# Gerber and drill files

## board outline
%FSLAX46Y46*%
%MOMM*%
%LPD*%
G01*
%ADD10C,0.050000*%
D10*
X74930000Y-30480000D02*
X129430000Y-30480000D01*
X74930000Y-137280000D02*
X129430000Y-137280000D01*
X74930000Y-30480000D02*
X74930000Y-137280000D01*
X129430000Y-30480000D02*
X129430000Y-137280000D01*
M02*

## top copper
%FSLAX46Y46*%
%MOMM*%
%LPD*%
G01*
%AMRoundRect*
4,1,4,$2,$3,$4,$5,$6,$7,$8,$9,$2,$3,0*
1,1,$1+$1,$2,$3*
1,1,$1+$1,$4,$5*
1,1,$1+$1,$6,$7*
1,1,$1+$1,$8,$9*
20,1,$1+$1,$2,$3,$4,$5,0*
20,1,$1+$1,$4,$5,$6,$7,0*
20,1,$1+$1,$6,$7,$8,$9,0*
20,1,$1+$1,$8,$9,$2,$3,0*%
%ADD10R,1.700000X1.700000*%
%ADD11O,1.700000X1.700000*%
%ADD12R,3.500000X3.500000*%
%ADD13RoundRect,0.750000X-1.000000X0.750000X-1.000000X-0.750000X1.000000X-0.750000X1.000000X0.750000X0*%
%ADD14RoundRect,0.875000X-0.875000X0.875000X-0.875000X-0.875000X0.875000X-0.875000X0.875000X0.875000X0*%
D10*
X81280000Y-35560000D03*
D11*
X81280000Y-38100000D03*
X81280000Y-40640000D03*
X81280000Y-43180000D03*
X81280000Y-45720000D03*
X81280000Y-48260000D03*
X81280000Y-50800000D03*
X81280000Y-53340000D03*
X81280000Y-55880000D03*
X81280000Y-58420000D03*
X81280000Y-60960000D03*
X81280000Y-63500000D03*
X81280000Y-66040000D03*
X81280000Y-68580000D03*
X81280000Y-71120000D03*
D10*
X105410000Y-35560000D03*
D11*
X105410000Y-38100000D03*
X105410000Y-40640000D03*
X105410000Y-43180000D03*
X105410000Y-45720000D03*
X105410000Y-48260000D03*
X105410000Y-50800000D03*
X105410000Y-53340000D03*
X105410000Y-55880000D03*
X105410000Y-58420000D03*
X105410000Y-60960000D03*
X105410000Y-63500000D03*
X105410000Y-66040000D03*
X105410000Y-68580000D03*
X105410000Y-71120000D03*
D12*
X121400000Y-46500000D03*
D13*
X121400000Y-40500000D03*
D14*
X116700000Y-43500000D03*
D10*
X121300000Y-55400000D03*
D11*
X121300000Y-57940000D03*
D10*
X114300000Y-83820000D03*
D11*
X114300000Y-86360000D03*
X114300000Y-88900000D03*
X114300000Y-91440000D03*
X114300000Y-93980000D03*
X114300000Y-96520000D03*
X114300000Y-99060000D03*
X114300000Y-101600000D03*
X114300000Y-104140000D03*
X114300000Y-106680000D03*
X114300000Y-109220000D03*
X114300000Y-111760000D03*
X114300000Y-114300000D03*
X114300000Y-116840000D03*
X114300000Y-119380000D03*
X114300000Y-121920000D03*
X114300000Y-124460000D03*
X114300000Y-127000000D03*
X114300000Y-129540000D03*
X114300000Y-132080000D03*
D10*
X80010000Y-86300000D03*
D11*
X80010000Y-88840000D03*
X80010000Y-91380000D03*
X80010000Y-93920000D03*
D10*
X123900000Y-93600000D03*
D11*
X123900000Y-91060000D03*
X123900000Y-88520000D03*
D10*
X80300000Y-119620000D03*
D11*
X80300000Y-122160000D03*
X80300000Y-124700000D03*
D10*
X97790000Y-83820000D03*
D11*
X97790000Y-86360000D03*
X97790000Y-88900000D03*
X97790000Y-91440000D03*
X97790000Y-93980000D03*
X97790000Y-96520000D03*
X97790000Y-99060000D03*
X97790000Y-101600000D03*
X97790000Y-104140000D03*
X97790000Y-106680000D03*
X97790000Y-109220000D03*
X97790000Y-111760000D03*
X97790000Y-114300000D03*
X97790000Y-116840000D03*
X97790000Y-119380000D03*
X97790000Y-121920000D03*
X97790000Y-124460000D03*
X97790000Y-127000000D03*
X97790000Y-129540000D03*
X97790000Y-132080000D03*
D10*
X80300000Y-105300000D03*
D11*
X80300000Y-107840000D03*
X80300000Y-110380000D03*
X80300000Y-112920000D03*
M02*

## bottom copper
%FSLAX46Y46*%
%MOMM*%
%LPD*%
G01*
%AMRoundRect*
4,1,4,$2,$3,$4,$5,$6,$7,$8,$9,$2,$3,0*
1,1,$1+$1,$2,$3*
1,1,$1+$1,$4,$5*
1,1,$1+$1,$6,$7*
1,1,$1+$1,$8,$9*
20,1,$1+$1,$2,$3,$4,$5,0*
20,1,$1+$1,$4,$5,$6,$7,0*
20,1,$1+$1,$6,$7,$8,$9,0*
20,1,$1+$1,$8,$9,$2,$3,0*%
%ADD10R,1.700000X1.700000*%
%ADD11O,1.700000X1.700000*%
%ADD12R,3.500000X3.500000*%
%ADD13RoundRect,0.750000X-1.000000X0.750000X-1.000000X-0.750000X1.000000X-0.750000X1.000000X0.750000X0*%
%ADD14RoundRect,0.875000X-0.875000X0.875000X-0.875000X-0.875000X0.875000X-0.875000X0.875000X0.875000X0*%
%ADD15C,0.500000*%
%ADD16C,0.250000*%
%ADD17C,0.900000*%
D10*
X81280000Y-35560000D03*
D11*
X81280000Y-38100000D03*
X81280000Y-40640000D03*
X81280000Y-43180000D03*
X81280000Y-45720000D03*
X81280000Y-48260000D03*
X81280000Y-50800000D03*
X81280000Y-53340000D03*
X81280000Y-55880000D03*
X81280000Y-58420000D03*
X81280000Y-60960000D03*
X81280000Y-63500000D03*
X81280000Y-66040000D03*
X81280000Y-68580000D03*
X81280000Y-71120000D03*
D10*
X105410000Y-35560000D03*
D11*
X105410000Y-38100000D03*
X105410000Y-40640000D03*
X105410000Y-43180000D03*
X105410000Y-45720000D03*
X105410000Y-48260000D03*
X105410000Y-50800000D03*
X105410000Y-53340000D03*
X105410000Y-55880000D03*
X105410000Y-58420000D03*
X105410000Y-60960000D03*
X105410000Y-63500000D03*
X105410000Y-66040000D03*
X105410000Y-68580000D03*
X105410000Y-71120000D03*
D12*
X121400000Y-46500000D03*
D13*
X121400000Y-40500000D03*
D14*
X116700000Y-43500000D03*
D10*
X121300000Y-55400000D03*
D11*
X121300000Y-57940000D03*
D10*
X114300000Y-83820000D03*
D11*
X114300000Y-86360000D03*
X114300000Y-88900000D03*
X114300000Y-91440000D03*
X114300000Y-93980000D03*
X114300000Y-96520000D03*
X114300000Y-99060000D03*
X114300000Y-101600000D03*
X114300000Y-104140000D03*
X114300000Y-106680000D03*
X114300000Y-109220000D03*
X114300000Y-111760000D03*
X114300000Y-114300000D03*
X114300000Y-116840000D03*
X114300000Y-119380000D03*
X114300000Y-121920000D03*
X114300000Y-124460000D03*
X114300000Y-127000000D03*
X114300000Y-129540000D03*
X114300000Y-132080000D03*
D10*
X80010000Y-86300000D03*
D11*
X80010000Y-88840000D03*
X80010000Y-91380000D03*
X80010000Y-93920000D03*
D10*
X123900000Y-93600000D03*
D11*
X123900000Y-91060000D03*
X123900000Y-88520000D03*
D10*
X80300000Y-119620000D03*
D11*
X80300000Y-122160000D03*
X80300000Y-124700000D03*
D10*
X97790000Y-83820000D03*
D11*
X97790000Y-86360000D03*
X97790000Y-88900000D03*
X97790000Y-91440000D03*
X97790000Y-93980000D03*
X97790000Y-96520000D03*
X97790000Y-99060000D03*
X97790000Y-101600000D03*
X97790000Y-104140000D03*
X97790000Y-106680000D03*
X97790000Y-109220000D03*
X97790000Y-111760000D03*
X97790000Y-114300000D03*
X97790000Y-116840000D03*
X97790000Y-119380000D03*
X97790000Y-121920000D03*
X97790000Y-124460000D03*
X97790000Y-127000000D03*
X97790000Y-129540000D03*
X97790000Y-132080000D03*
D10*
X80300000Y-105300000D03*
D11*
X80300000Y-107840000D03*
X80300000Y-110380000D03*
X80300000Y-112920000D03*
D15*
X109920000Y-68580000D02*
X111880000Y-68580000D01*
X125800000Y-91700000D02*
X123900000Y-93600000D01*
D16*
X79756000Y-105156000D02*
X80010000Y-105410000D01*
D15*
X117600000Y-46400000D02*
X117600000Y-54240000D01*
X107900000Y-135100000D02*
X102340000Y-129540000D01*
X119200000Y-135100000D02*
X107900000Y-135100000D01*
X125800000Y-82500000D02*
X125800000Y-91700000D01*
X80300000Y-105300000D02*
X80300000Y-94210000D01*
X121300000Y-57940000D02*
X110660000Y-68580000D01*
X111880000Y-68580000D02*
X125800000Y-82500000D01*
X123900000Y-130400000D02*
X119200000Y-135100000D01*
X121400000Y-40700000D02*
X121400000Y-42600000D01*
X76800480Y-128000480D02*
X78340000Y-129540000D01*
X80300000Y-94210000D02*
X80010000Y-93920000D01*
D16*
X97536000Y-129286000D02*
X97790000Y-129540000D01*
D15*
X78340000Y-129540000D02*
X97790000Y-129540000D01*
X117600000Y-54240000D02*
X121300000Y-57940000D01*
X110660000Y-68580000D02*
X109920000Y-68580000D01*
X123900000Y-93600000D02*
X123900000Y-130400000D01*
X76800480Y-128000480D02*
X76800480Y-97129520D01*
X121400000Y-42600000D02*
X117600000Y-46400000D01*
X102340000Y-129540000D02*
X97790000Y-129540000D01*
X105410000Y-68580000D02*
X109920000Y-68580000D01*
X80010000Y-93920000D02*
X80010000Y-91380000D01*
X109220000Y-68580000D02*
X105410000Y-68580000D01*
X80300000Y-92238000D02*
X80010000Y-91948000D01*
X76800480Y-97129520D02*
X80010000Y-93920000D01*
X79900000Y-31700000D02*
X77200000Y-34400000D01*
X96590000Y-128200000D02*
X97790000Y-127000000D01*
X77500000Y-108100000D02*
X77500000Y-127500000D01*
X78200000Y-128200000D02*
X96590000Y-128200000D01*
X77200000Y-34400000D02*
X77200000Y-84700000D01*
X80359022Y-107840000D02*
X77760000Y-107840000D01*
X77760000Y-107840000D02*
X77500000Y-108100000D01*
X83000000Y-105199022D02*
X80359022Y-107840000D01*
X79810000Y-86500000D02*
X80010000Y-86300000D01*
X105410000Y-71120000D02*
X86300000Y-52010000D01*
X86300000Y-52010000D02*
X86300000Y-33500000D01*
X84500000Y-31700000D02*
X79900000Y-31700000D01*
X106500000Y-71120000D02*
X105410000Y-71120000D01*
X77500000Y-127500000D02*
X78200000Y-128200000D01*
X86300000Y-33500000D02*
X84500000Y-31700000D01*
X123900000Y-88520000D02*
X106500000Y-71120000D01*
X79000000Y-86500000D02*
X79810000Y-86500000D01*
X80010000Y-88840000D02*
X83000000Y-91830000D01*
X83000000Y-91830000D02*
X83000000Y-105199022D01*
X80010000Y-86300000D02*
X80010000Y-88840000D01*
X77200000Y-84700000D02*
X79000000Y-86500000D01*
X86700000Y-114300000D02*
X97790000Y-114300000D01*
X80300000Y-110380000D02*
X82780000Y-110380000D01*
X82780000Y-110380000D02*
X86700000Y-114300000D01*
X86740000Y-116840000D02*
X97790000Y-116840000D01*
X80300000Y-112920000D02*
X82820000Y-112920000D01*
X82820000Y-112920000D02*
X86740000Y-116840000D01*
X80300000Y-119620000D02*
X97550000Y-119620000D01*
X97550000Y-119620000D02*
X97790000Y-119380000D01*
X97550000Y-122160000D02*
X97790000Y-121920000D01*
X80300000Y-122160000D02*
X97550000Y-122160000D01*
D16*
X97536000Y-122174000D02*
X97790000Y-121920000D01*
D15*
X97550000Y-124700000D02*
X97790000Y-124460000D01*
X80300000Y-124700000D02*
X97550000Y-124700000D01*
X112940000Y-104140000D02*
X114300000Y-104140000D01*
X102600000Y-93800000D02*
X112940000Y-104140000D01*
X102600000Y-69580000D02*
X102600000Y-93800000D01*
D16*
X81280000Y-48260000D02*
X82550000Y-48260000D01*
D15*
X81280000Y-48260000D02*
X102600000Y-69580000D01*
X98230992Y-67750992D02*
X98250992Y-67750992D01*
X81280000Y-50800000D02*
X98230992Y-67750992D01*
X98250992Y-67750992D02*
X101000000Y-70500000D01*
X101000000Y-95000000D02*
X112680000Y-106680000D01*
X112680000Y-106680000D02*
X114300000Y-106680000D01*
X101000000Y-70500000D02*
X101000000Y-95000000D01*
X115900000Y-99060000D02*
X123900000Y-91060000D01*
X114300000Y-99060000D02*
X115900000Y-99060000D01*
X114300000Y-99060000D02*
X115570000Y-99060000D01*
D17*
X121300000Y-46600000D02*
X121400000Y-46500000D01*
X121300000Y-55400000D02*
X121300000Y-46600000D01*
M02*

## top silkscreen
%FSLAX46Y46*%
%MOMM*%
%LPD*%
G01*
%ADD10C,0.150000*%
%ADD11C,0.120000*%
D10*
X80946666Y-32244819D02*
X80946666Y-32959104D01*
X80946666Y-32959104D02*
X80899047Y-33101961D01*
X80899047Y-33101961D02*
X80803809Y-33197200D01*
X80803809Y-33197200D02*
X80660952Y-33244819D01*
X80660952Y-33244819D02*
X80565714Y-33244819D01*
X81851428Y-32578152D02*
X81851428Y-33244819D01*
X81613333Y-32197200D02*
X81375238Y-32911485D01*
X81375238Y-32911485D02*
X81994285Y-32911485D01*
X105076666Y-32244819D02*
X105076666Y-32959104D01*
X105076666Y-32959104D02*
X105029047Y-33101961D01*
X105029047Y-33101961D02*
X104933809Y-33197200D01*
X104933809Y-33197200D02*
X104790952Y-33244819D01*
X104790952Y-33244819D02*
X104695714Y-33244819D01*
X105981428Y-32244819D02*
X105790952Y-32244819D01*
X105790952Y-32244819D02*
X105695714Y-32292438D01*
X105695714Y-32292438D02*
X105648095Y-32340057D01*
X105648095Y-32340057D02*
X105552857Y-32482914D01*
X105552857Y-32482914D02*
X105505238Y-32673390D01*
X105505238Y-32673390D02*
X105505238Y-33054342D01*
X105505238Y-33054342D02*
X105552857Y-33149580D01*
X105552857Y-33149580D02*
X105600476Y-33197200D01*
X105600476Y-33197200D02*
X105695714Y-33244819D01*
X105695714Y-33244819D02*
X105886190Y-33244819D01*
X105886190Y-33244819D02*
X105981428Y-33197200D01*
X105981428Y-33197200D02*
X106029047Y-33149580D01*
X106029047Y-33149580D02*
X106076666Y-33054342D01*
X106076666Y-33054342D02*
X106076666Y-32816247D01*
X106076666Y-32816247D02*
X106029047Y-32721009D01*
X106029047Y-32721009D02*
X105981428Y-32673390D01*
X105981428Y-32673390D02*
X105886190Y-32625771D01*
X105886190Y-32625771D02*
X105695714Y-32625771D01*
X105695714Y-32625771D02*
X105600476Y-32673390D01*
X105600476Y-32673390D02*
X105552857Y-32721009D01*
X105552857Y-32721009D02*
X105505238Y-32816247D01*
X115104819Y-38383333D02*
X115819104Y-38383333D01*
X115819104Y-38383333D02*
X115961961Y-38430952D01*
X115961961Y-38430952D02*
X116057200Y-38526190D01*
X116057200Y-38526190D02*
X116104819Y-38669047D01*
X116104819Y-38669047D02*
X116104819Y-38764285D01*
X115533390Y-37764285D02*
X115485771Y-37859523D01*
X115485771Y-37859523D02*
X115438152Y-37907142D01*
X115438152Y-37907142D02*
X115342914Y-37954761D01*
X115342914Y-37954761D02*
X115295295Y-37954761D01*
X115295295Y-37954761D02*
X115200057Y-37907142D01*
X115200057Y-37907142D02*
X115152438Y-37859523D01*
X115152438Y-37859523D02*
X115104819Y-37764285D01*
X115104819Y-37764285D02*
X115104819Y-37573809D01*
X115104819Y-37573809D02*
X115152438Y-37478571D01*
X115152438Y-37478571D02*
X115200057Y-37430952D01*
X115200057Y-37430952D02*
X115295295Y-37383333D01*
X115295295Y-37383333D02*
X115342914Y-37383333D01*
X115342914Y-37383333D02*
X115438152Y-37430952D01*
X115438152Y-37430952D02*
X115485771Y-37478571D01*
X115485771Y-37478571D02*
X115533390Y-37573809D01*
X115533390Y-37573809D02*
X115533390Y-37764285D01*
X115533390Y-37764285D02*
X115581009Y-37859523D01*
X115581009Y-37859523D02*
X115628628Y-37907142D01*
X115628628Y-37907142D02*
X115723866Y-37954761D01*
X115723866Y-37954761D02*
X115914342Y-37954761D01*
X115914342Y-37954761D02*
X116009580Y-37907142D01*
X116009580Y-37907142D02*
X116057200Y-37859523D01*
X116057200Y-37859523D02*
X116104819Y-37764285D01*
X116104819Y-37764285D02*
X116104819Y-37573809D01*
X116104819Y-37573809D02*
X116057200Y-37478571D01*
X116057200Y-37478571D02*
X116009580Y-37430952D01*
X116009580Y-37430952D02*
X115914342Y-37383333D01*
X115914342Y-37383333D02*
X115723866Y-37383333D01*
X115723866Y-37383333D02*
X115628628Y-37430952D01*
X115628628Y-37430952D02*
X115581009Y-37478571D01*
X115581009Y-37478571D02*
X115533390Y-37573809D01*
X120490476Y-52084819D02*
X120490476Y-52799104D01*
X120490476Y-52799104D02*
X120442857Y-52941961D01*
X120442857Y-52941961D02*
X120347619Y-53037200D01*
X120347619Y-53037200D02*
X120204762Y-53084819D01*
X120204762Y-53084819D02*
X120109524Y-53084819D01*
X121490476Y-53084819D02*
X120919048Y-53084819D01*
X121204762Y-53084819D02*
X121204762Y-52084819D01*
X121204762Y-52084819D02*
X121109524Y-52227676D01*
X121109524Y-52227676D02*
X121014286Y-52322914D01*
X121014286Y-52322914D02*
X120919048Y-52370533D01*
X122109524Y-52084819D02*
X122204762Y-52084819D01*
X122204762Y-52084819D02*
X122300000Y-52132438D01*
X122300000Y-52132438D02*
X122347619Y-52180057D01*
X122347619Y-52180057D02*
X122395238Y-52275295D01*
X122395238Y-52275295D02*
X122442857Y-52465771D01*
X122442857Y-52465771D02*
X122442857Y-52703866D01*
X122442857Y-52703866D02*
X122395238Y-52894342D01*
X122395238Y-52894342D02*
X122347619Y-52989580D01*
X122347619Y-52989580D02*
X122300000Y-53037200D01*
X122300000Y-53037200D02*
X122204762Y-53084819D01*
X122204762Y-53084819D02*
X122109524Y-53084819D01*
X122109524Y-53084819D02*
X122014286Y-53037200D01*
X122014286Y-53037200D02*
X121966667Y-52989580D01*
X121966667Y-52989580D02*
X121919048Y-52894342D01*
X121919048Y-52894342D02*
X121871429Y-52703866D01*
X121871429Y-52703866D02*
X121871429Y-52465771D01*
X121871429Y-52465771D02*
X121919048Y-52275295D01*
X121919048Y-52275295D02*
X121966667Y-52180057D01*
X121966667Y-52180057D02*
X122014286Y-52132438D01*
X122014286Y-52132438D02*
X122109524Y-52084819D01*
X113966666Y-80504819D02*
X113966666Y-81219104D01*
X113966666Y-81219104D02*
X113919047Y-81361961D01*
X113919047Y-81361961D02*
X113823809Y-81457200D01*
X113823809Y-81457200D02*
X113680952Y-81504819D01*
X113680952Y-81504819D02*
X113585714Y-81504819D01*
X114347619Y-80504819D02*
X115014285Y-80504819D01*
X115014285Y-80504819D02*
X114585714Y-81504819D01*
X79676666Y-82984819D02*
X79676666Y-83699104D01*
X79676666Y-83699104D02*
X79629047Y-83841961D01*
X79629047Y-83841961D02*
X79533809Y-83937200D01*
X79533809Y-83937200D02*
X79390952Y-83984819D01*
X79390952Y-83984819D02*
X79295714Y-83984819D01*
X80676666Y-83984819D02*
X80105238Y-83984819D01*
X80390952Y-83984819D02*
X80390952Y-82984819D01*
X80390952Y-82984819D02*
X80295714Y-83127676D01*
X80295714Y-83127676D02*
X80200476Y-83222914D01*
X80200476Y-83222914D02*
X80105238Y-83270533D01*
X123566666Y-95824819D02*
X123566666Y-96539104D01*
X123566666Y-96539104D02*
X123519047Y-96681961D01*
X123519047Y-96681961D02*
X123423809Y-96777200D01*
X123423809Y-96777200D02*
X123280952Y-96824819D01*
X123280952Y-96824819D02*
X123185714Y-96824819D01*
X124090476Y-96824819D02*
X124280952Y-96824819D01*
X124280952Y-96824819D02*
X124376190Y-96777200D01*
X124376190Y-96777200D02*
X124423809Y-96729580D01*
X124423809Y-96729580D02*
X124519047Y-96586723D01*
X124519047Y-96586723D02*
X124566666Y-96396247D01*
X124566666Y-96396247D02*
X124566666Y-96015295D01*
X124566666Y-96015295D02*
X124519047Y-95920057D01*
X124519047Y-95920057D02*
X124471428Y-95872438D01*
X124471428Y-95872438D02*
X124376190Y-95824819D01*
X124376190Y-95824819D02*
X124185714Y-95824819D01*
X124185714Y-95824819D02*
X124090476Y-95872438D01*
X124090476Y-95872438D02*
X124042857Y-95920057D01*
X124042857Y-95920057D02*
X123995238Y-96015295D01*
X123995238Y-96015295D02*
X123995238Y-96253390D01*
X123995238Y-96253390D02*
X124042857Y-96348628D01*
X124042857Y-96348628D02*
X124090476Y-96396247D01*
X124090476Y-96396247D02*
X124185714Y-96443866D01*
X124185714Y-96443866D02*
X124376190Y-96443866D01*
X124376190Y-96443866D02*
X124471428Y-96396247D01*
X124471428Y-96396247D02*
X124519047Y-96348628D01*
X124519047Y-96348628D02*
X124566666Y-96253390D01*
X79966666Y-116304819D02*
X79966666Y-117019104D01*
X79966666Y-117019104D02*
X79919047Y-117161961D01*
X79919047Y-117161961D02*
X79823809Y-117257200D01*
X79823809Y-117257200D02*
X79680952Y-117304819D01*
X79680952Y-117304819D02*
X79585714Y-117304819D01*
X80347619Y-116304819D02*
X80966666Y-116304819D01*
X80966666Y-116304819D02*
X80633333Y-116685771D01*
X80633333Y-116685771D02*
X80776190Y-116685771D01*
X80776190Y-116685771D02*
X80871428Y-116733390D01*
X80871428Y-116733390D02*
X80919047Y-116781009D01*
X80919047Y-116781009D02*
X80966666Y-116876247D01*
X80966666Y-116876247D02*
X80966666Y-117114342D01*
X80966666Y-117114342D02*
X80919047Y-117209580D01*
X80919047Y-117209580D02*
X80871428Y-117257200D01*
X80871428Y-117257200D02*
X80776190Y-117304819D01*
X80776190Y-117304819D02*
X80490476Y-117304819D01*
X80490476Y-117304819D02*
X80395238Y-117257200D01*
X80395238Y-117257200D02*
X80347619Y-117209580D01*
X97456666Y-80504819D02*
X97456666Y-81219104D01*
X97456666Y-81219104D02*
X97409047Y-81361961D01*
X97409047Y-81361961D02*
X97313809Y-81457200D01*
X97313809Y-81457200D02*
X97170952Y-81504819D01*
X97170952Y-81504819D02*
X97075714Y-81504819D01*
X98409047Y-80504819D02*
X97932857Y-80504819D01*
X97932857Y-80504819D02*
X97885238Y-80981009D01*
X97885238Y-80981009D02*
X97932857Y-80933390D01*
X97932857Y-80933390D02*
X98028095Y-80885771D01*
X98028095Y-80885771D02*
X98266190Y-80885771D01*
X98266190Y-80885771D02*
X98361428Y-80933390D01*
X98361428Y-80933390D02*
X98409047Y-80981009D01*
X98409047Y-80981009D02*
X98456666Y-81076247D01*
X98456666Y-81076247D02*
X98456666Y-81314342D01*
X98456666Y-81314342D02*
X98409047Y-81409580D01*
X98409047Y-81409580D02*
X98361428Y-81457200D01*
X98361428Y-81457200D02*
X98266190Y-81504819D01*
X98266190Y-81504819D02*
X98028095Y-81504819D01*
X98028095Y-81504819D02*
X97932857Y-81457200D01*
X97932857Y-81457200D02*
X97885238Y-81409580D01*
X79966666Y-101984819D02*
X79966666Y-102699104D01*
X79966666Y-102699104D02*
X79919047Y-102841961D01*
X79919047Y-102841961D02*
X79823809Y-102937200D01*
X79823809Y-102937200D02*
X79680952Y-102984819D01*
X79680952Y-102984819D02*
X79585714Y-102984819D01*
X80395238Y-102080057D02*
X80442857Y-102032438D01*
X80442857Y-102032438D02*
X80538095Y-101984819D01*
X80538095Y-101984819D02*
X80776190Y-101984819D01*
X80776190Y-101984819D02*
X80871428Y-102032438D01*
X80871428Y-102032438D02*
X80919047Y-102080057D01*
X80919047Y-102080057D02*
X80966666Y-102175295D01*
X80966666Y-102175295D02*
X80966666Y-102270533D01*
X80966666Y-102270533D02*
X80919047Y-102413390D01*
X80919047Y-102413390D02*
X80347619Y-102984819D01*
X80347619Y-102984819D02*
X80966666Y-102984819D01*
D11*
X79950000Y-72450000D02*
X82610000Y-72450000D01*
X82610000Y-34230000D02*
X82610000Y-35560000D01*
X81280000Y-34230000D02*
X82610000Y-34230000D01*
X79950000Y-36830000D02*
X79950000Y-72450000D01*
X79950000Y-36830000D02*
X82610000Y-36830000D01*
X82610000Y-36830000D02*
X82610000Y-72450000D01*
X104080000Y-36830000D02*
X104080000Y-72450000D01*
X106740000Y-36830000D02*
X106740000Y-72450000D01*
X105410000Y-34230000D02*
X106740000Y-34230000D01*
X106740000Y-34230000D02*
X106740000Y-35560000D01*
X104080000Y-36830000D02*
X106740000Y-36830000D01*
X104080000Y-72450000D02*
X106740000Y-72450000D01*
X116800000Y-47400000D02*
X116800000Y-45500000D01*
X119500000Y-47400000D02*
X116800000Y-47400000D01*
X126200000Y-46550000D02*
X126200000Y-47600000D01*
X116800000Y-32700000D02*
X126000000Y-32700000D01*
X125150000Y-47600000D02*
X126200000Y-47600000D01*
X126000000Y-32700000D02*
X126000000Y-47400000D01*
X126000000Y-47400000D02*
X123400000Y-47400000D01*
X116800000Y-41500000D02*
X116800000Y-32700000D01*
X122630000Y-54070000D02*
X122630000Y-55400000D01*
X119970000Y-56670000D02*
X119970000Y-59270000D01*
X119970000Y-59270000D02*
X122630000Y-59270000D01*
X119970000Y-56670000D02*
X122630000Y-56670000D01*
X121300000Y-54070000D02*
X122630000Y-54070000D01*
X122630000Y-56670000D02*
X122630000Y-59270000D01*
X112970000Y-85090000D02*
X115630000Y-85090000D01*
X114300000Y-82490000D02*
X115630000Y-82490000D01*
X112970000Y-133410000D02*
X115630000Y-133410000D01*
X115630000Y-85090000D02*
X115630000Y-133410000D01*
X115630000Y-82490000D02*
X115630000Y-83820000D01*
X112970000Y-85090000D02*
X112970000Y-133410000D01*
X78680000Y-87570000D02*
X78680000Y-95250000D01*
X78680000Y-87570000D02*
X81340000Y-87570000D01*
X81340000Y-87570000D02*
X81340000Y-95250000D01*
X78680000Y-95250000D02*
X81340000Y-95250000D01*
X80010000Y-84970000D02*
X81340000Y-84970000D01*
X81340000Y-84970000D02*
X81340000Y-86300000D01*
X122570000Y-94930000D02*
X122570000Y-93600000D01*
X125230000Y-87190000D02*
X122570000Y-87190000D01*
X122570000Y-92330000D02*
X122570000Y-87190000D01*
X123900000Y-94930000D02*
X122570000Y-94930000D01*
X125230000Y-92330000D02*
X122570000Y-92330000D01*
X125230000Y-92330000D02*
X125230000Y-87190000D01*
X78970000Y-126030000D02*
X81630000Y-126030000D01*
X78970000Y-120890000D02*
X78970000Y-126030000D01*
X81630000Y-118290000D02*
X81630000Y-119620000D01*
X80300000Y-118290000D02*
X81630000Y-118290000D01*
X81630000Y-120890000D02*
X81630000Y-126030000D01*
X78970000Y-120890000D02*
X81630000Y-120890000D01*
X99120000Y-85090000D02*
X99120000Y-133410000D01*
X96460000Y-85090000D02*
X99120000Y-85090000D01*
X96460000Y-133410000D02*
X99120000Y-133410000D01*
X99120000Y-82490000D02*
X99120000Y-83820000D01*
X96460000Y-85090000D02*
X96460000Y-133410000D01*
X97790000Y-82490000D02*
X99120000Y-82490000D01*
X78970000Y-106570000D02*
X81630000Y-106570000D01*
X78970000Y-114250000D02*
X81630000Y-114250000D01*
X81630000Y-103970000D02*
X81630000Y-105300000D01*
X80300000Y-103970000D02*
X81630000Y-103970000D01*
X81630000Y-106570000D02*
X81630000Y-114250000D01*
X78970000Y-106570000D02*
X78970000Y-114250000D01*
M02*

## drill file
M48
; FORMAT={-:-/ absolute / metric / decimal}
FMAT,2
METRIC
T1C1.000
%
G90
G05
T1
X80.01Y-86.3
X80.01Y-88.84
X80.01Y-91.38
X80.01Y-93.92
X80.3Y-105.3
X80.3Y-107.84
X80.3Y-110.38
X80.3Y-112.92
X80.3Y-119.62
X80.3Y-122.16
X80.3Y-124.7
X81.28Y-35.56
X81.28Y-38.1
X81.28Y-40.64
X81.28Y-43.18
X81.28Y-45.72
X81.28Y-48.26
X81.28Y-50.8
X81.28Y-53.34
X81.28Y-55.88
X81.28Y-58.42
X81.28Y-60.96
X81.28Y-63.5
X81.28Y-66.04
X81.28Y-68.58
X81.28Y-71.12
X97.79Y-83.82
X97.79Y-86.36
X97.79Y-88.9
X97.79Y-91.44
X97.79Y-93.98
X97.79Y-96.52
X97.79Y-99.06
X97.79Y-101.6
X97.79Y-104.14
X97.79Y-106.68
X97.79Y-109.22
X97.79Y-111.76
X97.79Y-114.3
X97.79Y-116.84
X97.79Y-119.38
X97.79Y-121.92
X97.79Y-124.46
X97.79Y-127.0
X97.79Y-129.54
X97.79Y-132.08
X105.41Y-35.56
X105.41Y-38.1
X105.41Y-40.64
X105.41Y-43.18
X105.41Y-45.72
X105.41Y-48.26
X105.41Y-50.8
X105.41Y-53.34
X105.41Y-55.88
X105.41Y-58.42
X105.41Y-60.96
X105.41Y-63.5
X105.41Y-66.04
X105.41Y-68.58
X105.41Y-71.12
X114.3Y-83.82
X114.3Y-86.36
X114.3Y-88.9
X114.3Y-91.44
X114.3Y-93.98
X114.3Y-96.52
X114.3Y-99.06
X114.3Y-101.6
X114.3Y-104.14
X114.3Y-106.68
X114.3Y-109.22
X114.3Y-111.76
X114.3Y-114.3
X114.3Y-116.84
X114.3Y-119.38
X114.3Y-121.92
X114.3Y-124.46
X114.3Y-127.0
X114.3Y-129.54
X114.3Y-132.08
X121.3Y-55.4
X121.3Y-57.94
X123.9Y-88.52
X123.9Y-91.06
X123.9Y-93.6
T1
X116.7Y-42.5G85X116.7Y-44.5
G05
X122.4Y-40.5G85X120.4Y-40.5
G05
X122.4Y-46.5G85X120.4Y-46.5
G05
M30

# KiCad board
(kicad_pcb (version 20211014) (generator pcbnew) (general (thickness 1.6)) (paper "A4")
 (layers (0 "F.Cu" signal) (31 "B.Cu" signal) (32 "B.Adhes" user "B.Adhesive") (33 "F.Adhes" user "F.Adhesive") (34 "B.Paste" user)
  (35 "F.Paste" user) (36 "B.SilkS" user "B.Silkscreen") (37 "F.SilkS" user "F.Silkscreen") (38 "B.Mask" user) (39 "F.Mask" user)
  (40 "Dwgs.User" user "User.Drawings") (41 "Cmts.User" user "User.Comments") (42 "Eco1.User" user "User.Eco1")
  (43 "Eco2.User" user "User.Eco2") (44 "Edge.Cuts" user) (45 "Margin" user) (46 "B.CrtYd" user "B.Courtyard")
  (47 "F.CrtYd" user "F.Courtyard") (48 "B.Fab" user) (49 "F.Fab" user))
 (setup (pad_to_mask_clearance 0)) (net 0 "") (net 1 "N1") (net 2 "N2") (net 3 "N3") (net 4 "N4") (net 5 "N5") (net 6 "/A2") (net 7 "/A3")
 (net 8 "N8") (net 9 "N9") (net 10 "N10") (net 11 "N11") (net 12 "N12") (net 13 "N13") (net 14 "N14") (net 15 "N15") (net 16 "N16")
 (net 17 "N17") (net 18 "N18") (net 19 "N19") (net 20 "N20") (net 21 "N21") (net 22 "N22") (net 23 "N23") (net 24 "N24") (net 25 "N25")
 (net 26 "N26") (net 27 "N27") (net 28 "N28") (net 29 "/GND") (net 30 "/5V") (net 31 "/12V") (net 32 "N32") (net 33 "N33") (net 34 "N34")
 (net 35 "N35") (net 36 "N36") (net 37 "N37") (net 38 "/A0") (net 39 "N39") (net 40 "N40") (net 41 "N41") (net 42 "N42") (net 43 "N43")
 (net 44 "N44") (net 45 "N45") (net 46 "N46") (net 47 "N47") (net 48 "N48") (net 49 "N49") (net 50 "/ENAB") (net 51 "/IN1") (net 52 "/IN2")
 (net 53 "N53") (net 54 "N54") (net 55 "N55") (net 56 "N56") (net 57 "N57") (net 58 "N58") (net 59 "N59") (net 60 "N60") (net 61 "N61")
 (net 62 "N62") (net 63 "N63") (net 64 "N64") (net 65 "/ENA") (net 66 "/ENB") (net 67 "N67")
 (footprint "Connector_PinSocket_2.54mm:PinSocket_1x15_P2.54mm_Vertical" (layer "F.Cu") (at 81.28 35.56)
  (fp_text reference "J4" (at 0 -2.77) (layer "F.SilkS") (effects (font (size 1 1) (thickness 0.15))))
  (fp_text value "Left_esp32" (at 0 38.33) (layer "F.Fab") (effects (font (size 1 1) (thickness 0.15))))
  (fp_line (start -1.33 36.89) (end 1.33 36.89) (layer "F.SilkS") (width 0.12))
  (fp_line (start 1.33 -1.33) (end 1.33 0) (layer "F.SilkS") (width 0.12))
  (fp_line (start 0 -1.33) (end 1.33 -1.33) (layer "F.SilkS") (width 0.12))
  (fp_line (start -1.33 1.27) (end -1.33 36.89) (layer "F.SilkS") (width 0.12))
  (fp_line (start -1.33 1.27) (end 1.33 1.27) (layer "F.SilkS") (width 0.12))
  (fp_line (start 1.33 1.27) (end 1.33 36.89) (layer "F.SilkS") (width 0.12))
  (pad "1" thru_hole rect locked (at 0 0) (size 1.7 1.7) (drill 1) (layers *.Cu *.Mask) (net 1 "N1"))
  (pad "2" thru_hole oval locked (at 0 2.54) (size 1.7 1.7) (drill 1) (layers *.Cu *.Mask) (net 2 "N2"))
  (pad "3" thru_hole oval locked (at 0 5.08) (size 1.7 1.7) (drill 1) (layers *.Cu *.Mask) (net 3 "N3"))
  (pad "4" thru_hole oval locked (at 0 7.62) (size 1.7 1.7) (drill 1) (layers *.Cu *.Mask) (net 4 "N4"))
  (pad "5" thru_hole oval locked (at 0 10.16) (size 1.7 1.7) (drill 1) (layers *.Cu *.Mask) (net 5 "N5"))
  (pad "6" thru_hole oval locked (at 0 12.7) (size 1.7 1.7) (drill 1) (layers *.Cu *.Mask) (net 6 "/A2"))
  (pad "7" thru_hole oval locked (at 0 15.24) (size 1.7 1.7) (drill 1) (layers *.Cu *.Mask) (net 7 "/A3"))
  (pad "8" thru_hole oval locked (at 0 17.78) (size 1.7 1.7) (drill 1) (layers *.Cu *.Mask) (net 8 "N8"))
  (pad "9" thru_hole oval locked (at 0 20.32) (size 1.7 1.7) (drill 1) (layers *.Cu *.Mask) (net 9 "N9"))
  (pad "10" thru_hole oval locked (at 0 22.86) (size 1.7 1.7) (drill 1) (layers *.Cu *.Mask) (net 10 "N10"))
  (pad "11" thru_hole oval locked (at 0 25.4) (size 1.7 1.7) (drill 1) (layers *.Cu *.Mask) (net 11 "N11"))
  (pad "12" thru_hole oval locked (at 0 27.94) (size 1.7 1.7) (drill 1) (layers *.Cu *.Mask) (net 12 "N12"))
  (pad "13" thru_hole oval locked (at 0 30.48) (size 1.7 1.7) (drill 1) (layers *.Cu *.Mask) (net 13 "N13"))
  (pad "14" thru_hole oval locked (at 0 33.02) (size 1.7 1.7) (drill 1) (layers *.Cu *.Mask) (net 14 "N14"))
  (pad "15" thru_hole oval locked (at 0 35.56) (size 1.7 1.7) (drill 1) (layers *.Cu *.Mask) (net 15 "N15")))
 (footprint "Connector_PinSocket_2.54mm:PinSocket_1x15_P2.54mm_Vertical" (layer "F.Cu") (at 105.41 35.56)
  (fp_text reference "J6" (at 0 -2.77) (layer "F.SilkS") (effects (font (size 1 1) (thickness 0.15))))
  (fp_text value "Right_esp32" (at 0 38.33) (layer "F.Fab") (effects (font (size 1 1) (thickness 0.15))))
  (fp_line (start -1.33 1.27) (end -1.33 36.89) (layer "F.SilkS") (width 0.12))
  (fp_line (start 1.33 1.27) (end 1.33 36.89) (layer "F.SilkS") (width 0.12))
  (fp_line (start 0 -1.33) (end 1.33 -1.33) (layer "F.SilkS") (width 0.12))
  (fp_line (start 1.33 -1.33) (end 1.33 0) (layer "F.SilkS") (width 0.12))
  (fp_line (start -1.33 1.27) (end 1.33 1.27) (layer "F.SilkS") (width 0.12))
  (fp_line (start -1.33 36.89) (end 1.33 36.89) (layer "F.SilkS") (width 0.12))
  (pad "1" thru_hole rect locked (at 0 0) (size 1.7 1.7) (drill 1) (layers *.Cu *.Mask) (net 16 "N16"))
  (pad "2" thru_hole oval locked (at 0 2.54) (size 1.7 1.7) (drill 1) (layers *.Cu *.Mask) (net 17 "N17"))
  (pad "3" thru_hole oval locked (at 0 5.08) (size 1.7 1.7) (drill 1) (layers *.Cu *.Mask) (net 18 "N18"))
  (pad "4" thru_hole oval locked (at 0 7.62) (size 1.7 1.7) (drill 1) (layers *.Cu *.Mask) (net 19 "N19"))
  (pad "5" thru_hole oval locked (at 0 10.16) (size 1.7 1.7) (drill 1) (layers *.Cu *.Mask) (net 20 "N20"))
  (pad "6" thru_hole oval locked (at 0 12.7) (size 1.7 1.7) (drill 1) (layers *.Cu *.Mask) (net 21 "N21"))
  (pad "7" thru_hole oval locked (at 0 15.24) (size 1.7 1.7) (drill 1) (layers *.Cu *.Mask) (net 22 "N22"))
  (pad "8" thru_hole oval locked (at 0 17.78) (size 1.7 1.7) (drill 1) (layers *.Cu *.Mask) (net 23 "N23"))
  (pad "9" thru_hole oval locked (at 0 20.32) (size 1.7 1.7) (drill 1) (layers *.Cu *.Mask) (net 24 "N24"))
  (pad "10" thru_hole oval locked (at 0 22.86) (size 1.7 1.7) (drill 1) (layers *.Cu *.Mask) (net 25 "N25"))
  (pad "11" thru_hole oval locked (at 0 25.4) (size 1.7 1.7) (drill 1) (layers *.Cu *.Mask) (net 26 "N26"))
  (pad "12" thru_hole oval locked (at 0 27.94) (size 1.7 1.7) (drill 1) (layers *.Cu *.Mask) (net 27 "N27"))
  (pad "13" thru_hole oval locked (at 0 30.48) (size 1.7 1.7) (drill 1) (layers *.Cu *.Mask) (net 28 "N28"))
  (pad "14" thru_hole oval locked (at 0 33.02) (size 1.7 1.7) (drill 1) (layers *.Cu *.Mask) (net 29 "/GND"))
  (pad "15" thru_hole oval locked (at 0 35.56) (size 1.7 1.7) (drill 1) (layers *.Cu *.Mask) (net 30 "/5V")))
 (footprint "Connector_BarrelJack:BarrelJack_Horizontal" (layer "F.Cu") (at 121.4 46.5 -90)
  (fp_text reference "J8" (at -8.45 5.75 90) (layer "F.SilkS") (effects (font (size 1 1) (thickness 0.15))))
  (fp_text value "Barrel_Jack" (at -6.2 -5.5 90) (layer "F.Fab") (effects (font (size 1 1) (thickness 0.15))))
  (fp_line (start 0.9 4.6) (end -1 4.6) (layer "F.SilkS") (width 0.12))
  (fp_line (start 0.9 1.9) (end 0.9 4.6) (layer "F.SilkS") (width 0.12))
  (fp_line (start 0.05 -4.8) (end 1.1 -4.8) (layer "F.SilkS") (width 0.12))
  (fp_line (start -13.8 4.6) (end -13.8 -4.6) (layer "F.SilkS") (width 0.12))
  (fp_line (start 1.1 -3.75) (end 1.1 -4.8) (layer "F.SilkS") (width 0.12))
  (fp_line (start -13.8 -4.6) (end 0.9 -4.6) (layer "F.SilkS") (width 0.12))
  (fp_line (start 0.9 -4.6) (end 0.9 -2) (layer "F.SilkS") (width 0.12))
  (fp_line (start -5 4.6) (end -13.8 4.6) (layer "F.SilkS") (width 0.12))
  (pad "1" thru_hole rect (at 0 0 270) (size 3.5 3.5) (drill oval 1 3) (layers *.Cu *.Mask) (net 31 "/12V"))
  (pad "2" thru_hole roundrect (at -6 0 270) (size 3 3.5) (drill oval 1 3) (layers *.Cu *.Mask) (roundrect_rratio 0.25) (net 29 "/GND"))
  (pad "3" thru_hole roundrect (at -3 4.7 270) (size 3.5 3.5) (drill oval 3 1) (layers *.Cu *.Mask) (roundrect_rratio 0.25)))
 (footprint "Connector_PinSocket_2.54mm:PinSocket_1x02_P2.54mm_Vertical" (layer "F.Cu") (at 121.3 55.4)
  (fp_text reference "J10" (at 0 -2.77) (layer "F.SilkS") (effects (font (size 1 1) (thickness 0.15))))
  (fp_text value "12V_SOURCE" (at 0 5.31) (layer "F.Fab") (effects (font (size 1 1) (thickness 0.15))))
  (fp_line (start 1.33 -1.33) (end 1.33 0) (layer "F.SilkS") (width 0.12))
  (fp_line (start -1.33 1.27) (end -1.33 3.87) (layer "F.SilkS") (width 0.12))
  (fp_line (start -1.33 3.87) (end 1.33 3.87) (layer "F.SilkS") (width 0.12))
  (fp_line (start -1.33 1.27) (end 1.33 1.27) (layer "F.SilkS") (width 0.12))
  (fp_line (start 0 -1.33) (end 1.33 -1.33) (layer "F.SilkS") (width 0.12))
  (fp_line (start 1.33 1.27) (end 1.33 3.87) (layer "F.SilkS") (width 0.12))
  (pad "1" thru_hole rect locked (at 0 0) (size 1.7 1.7) (drill 1) (layers *.Cu *.Mask) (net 31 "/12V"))
  (pad "2" thru_hole oval locked (at 0 2.54) (size 1.7 1.7) (drill 1) (layers *.Cu *.Mask) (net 29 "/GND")))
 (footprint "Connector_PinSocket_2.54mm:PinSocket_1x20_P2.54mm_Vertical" (layer "F.Cu") (at 114.3 83.82)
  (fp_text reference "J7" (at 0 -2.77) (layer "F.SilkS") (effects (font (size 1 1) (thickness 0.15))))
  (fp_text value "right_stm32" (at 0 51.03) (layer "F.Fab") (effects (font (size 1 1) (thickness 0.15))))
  (fp_line (start -1.33 1.27) (end 1.33 1.27) (layer "F.SilkS") (width 0.12))
  (fp_line (start 0 -1.33) (end 1.33 -1.33) (layer "F.SilkS") (width 0.12))
  (fp_line (start -1.33 49.59) (end 1.33 49.59) (layer "F.SilkS") (width 0.12))
  (fp_line (start 1.33 1.27) (end 1.33 49.59) (layer "F.SilkS") (width 0.12))
  (fp_line (start 1.33 -1.33) (end 1.33 0) (layer "F.SilkS") (width 0.12))
  (fp_line (start -1.33 1.27) (end -1.33 49.59) (layer "F.SilkS") (width 0.12))
  (pad "1" thru_hole rect locked (at 0 0) (size 1.7 1.7) (drill 1) (layers *.Cu *.Mask) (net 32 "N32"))
  (pad "2" thru_hole oval locked (at 0 2.54) (size 1.7 1.7) (drill 1) (layers *.Cu *.Mask) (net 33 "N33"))
  (pad "3" thru_hole oval locked (at 0 5.08) (size 1.7 1.7) (drill 1) (layers *.Cu *.Mask) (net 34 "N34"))
  (pad "4" thru_hole oval locked (at 0 7.62) (size 1.7 1.7) (drill 1) (layers *.Cu *.Mask) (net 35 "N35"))
  (pad "5" thru_hole oval locked (at 0 10.16) (size 1.7 1.7) (drill 1) (layers *.Cu *.Mask) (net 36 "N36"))
  (pad "6" thru_hole oval locked (at 0 12.7) (size 1.7 1.7) (drill 1) (layers *.Cu *.Mask) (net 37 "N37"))
  (pad "7" thru_hole oval locked (at 0 15.24) (size 1.7 1.7) (drill 1) (layers *.Cu *.Mask) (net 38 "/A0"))
  (pad "8" thru_hole oval locked (at 0 17.78) (size 1.7 1.7) (drill 1) (layers *.Cu *.Mask) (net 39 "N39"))
  (pad "9" thru_hole oval locked (at 0 20.32) (size 1.7 1.7) (drill 1) (layers *.Cu *.Mask) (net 6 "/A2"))
  (pad "10" thru_hole oval locked (at 0 22.86) (size 1.7 1.7) (drill 1) (layers *.Cu *.Mask) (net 7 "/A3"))
  (pad "11" thru_hole oval locked (at 0 25.4) (size 1.7 1.7) (drill 1) (layers *.Cu *.Mask) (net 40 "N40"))
  (pad "12" thru_hole oval locked (at 0 27.94) (size 1.7 1.7) (drill 1) (layers *.Cu *.Mask) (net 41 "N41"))
  (pad "13" thru_hole oval locked (at 0 30.48) (size 1.7 1.7) (drill 1) (layers *.Cu *.Mask) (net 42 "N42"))
  (pad "14" thru_hole oval locked (at 0 33.02) (size 1.7 1.7) (drill 1) (layers *.Cu *.Mask) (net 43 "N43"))
  (pad "15" thru_hole oval locked (at 0 35.56) (size 1.7 1.7) (drill 1) (layers *.Cu *.Mask) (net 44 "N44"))
  (pad "16" thru_hole oval locked (at 0 38.1) (size 1.7 1.7) (drill 1) (layers *.Cu *.Mask) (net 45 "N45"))
  (pad "17" thru_hole oval locked (at 0 40.64) (size 1.7 1.7) (drill 1) (layers *.Cu *.Mask) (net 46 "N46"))
  (pad "18" thru_hole oval locked (at 0 43.18) (size 1.7 1.7) (drill 1) (layers *.Cu *.Mask) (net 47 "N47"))
  (pad "19" thru_hole oval locked (at 0 45.72) (size 1.7 1.7) (drill 1) (layers *.Cu *.Mask) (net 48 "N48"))
  (pad "20" thru_hole oval locked (at 0 48.26) (size 1.7 1.7) (drill 1) (layers *.Cu *.Mask) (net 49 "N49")))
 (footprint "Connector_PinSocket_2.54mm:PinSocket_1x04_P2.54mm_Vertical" (layer "F.Cu") (at 80.01 86.3)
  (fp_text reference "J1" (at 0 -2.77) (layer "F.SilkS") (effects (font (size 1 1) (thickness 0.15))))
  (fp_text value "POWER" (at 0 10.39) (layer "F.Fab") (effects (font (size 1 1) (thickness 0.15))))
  (fp_line (start -1.33 1.27) (end -1.33 8.95) (layer "F.SilkS") (width 0.12))
  (fp_line (start -1.33 1.27) (end 1.33 1.27) (layer "F.SilkS") (width 0.12))
  (fp_line (start 1.33 1.27) (end 1.33 8.95) (layer "F.SilkS") (width 0.12))
  (fp_line (start -1.33 8.95) (end 1.33 8.95) (layer "F.SilkS") (width 0.12))
  (fp_line (start 0 -1.33) (end 1.33 -1.33) (layer "F.SilkS") (width 0.12))
  (fp_line (start 1.33 -1.33) (end 1.33 0) (layer "F.SilkS") (width 0.12))
  (pad "1" thru_hole rect locked (at 0 0) (size 1.7 1.7) (drill 1) (layers *.Cu *.Mask) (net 30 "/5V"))
  (pad "2" thru_hole oval locked (at 0 2.54) (size 1.7 1.7) (drill 1) (layers *.Cu *.Mask) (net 30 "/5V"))
  (pad "3" thru_hole oval locked (at 0 5.08) (size 1.7 1.7) (drill 1) (layers *.Cu *.Mask) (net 29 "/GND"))
  (pad "4" thru_hole oval locked (at 0 7.62) (size 1.7 1.7) (drill 1) (layers *.Cu *.Mask) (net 29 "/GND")))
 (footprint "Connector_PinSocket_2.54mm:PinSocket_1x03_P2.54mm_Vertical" (layer "F.Cu") (at 123.9 93.6 180)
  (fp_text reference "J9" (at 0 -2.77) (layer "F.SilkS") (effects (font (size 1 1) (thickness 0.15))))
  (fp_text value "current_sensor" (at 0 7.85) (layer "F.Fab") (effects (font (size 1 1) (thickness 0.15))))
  (fp_line (start 1.33 -1.33) (end 1.33 0) (layer "F.SilkS") (width 0.12))
  (fp_line (start -1.33 6.41) (end 1.33 6.41) (layer "F.SilkS") (width 0.12))
  (fp_line (start 1.33 1.27) (end 1.33 6.41) (layer "F.SilkS") (width 0.12))
  (fp_line (start 0 -1.33) (end 1.33 -1.33) (layer "F.SilkS") (width 0.12))
  (fp_line (start -1.33 1.27) (end 1.33 1.27) (layer "F.SilkS") (width 0.12))
  (fp_line (start -1.33 1.27) (end -1.33 6.41) (layer "F.SilkS") (width 0.12))
  (pad "1" thru_hole rect locked (at 0 0 180) (size 1.7 1.7) (drill 1) (layers *.Cu *.Mask) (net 29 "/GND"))
  (pad "2" thru_hole oval locked (at 0 2.54 180) (size 1.7 1.7) (drill 1) (layers *.Cu *.Mask) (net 38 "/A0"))
  (pad "3" thru_hole oval locked (at 0 5.08 180) (size 1.7 1.7) (drill 1) (layers *.Cu *.Mask) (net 30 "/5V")))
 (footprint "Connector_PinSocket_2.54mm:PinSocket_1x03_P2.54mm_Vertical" (layer "F.Cu") (at 80.3 119.62)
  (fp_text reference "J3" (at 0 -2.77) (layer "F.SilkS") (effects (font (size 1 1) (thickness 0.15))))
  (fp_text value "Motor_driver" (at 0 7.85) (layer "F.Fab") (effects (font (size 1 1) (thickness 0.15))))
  (fp_line (start -1.33 6.41) (end 1.33 6.41) (layer "F.SilkS") (width 0.12))
  (fp_line (start -1.33 1.27) (end -1.33 6.41) (layer "F.SilkS") (width 0.12))
  (fp_line (start 1.33 -1.33) (end 1.33 0) (layer "F.SilkS") (width 0.12))
  (fp_line (start 0 -1.33) (end 1.33 -1.33) (layer "F.SilkS") (width 0.12))
  (fp_line (start 1.33 1.27) (end 1.33 6.41) (layer "F.SilkS") (width 0.12))
  (fp_line (start -1.33 1.27) (end 1.33 1.27) (layer "F.SilkS") (width 0.12))
  (pad "1" thru_hole rect locked (at 0 0) (size 1.7 1.7) (drill 1) (layers *.Cu *.Mask) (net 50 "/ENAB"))
  (pad "2" thru_hole oval locked (at 0 2.54) (size 1.7 1.7) (drill 1) (layers *.Cu *.Mask) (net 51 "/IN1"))
  (pad "3" thru_hole oval locked (at 0 5.08) (size 1.7 1.7) (drill 1) (layers *.Cu *.Mask) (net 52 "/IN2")))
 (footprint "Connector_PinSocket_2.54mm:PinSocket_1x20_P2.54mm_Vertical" (layer "F.Cu") (at 97.79 83.82)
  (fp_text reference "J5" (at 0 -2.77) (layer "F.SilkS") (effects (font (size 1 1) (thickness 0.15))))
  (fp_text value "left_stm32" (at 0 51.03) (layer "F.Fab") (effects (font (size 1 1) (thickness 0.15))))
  (fp_line (start 1.33 1.27) (end 1.33 49.59) (layer "F.SilkS") (width 0.12))
  (fp_line (start -1.33 1.27) (end 1.33 1.27) (layer "F.SilkS") (width 0.12))
  (fp_line (start -1.33 49.59) (end 1.33 49.59) (layer "F.SilkS") (width 0.12))
  (fp_line (start 1.33 -1.33) (end 1.33 0) (layer "F.SilkS") (width 0.12))
  (fp_line (start -1.33 1.27) (end -1.33 49.59) (layer "F.SilkS") (width 0.12))
  (fp_line (start 0 -1.33) (end 1.33 -1.33) (layer "F.SilkS") (width 0.12))
  (pad "1" thru_hole rect locked (at 0 0) (size 1.7 1.7) (drill 1) (layers *.Cu *.Mask) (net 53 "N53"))
  (pad "2" thru_hole oval locked (at 0 2.54) (size 1.7 1.7) (drill 1) (layers *.Cu *.Mask) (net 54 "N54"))
  (pad "3" thru_hole oval locked (at 0 5.08) (size 1.7 1.7) (drill 1) (layers *.Cu *.Mask) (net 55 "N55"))
  (pad "4" thru_hole oval locked (at 0 7.62) (size 1.7 1.7) (drill 1) (layers *.Cu *.Mask) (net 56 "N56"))
  (pad "5" thru_hole oval locked (at 0 10.16) (size 1.7 1.7) (drill 1) (layers *.Cu *.Mask) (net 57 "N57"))
  (pad "6" thru_hole oval locked (at 0 12.7) (size 1.7 1.7) (drill 1) (layers *.Cu *.Mask) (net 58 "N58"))
  (pad "7" thru_hole oval locked (at 0 15.24) (size 1.7 1.7) (drill 1) (layers *.Cu *.Mask) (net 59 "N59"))
  (pad "8" thru_hole oval locked (at 0 17.78) (size 1.7 1.7) (drill 1) (layers *.Cu *.Mask) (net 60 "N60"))
  (pad "9" thru_hole oval locked (at 0 20.32) (size 1.7 1.7) (drill 1) (layers *.Cu *.Mask) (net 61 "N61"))
  (pad "10" thru_hole oval locked (at 0 22.86) (size 1.7 1.7) (drill 1) (layers *.Cu *.Mask) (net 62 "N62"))
  (pad "11" thru_hole oval locked (at 0 25.4) (size 1.7 1.7) (drill 1) (layers *.Cu *.Mask) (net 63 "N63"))
  (pad "12" thru_hole oval locked (at 0 27.94) (size 1.7 1.7) (drill 1) (layers *.Cu *.Mask) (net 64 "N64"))
  (pad "13" thru_hole oval locked (at 0 30.48) (size 1.7 1.7) (drill 1) (layers *.Cu *.Mask) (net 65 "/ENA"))
  (pad "14" thru_hole oval locked (at 0 33.02) (size 1.7 1.7) (drill 1) (layers *.Cu *.Mask) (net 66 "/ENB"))
  (pad "15" thru_hole oval locked (at 0 35.56) (size 1.7 1.7) (drill 1) (layers *.Cu *.Mask) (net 50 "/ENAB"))
  (pad "16" thru_hole oval locked (at 0 38.1) (size 1.7 1.7) (drill 1) (layers *.Cu *.Mask) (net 51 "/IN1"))
  (pad "17" thru_hole oval locked (at 0 40.64) (size 1.7 1.7) (drill 1) (layers *.Cu *.Mask) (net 52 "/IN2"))
  (pad "18" thru_hole oval locked (at 0 43.18) (size 1.7 1.7) (drill 1) (layers *.Cu *.Mask) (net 30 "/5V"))
  (pad "19" thru_hole oval locked (at 0 45.72) (size 1.7 1.7) (drill 1) (layers *.Cu *.Mask) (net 29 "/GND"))
  (pad "20" thru_hole oval locked (at 0 48.26) (size 1.7 1.7) (drill 1) (layers *.Cu *.Mask) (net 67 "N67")))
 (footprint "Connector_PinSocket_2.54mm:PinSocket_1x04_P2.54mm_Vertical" (layer "F.Cu") (at 80.3 105.3)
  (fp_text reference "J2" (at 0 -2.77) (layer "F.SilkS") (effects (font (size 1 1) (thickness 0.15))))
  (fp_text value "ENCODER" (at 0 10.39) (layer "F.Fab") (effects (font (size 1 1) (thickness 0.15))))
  (fp_line (start -1.33 1.27) (end 1.33 1.27) (layer "F.SilkS") (width 0.12))
  (fp_line (start -1.33 8.95) (end 1.33 8.95) (layer "F.SilkS") (width 0.12))
  (fp_line (start 1.33 -1.33) (end 1.33 0) (layer "F.SilkS") (width 0.12))
  (fp_line (start 0 -1.33) (end 1.33 -1.33) (layer "F.SilkS") (width 0.12))
  (fp_line (start 1.33 1.27) (end 1.33 8.95) (layer "F.SilkS") (width 0.12))
  (fp_line (start -1.33 1.27) (end -1.33 8.95) (layer "F.SilkS") (width 0.12))
  (pad "1" thru_hole rect locked (at 0 0) (size 1.7 1.7) (drill 1) (layers *.Cu *.Mask) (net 29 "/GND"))
  (pad "2" thru_hole oval locked (at 0 2.54) (size 1.7 1.7) (drill 1) (layers *.Cu *.Mask) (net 30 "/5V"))
  (pad "3" thru_hole oval locked (at 0 5.08) (size 1.7 1.7) (drill 1) (layers *.Cu *.Mask) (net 65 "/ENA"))
  (pad "4" thru_hole oval locked (at 0 7.62) (size 1.7 1.7) (drill 1) (layers *.Cu *.Mask) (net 66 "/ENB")))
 (gr_line (start 74.93 30.48) (end 129.43 30.48) (layer "Edge.Cuts") (width 0.05))
 (gr_line (start 74.93 137.28) (end 129.43 137.28) (layer "Edge.Cuts") (width 0.05))
 (gr_line (start 74.93 30.48) (end 74.93 137.28) (layer "Edge.Cuts") (width 0.05))
 (gr_line (start 129.43 30.48) (end 129.43 137.28) (layer "Edge.Cuts") (width 0.05))
 (segment (start 109.92 68.58) (end 111.88 68.58) (width 0.5) (layer "B.Cu") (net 29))
 (segment (start 125.8 91.7) (end 123.9 93.6) (width 0.5) (layer "B.Cu") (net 29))
 (segment (start 79.756 105.156) (end 80.01 105.41) (width 0.25) (layer "B.Cu") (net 29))
 (segment (start 117.6 46.4) (end 117.6 54.24) (width 0.5) (layer "B.Cu") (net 29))
 (segment (start 107.9 135.1) (end 102.34 129.54) (width 0.5) (layer "B.Cu") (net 29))
 (segment (start 119.2 135.1) (end 107.9 135.1) (width 0.5) (layer "B.Cu") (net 29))
 (segment (start 125.8 82.5) (end 125.8 91.7) (width 0.5) (layer "B.Cu") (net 29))
 (segment (start 80.3 105.3) (end 80.3 94.21) (width 0.5) (layer "B.Cu") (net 29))
 (segment (start 121.3 57.94) (end 110.66 68.58) (width 0.5) (layer "B.Cu") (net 29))
 (segment (start 111.88 68.58) (end 125.8 82.5) (width 0.5) (layer "B.Cu") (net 29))
 (segment (start 123.9 130.4) (end 119.2 135.1) (width 0.5) (layer "B.Cu") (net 29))
 (segment (start 121.4 40.7) (end 121.4 42.6) (width 0.5) (layer "B.Cu") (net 29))
 (segment (start 76.80048 128.00048) (end 78.34 129.54) (width 0.5) (layer "B.Cu") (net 29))
 (segment (start 80.3 94.21) (end 80.01 93.92) (width 0.5) (layer "B.Cu") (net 29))
 (segment (start 97.536 129.286) (end 97.79 129.54) (width 0.25) (layer "B.Cu") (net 29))
 (segment (start 78.34 129.54) (end 97.79 129.54) (width 0.5) (layer "B.Cu") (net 29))
 (segment (start 117.6 54.24) (end 121.3 57.94) (width 0.5) (layer "B.Cu") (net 29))
 (segment (start 110.66 68.58) (end 109.92 68.58) (width 0.5) (layer "B.Cu") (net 29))
 (segment (start 123.9 93.6) (end 123.9 130.4) (width 0.5) (layer "B.Cu") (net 29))
 (segment (start 76.80048 128.00048) (end 76.80048 97.12952) (width 0.5) (layer "B.Cu") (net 29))
 (segment (start 121.4 42.6) (end 117.6 46.4) (width 0.5) (layer "B.Cu") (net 29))
 (segment (start 102.34 129.54) (end 97.79 129.54) (width 0.5) (layer "B.Cu") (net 29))
 (segment (start 105.41 68.58) (end 109.92 68.58) (width 0.5) (layer "B.Cu") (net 29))
 (segment (start 80.01 93.92) (end 80.01 91.38) (width 0.5) (layer "B.Cu") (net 29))
 (segment (start 109.22 68.58) (end 105.41 68.58) (width 0.5) (layer "B.Cu") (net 29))
 (segment (start 80.3 92.238) (end 80.01 91.948) (width 0.5) (layer "B.Cu") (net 29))
 (segment (start 76.80048 97.12952) (end 80.01 93.92) (width 0.5) (layer "B.Cu") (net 29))
 (segment (start 79.9 31.7) (end 77.2 34.4) (width 0.5) (layer "B.Cu") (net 30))
 (segment (start 96.59 128.2) (end 97.79 127) (width 0.5) (layer "B.Cu") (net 30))
 (segment (start 77.5 108.1) (end 77.5 127.5) (width 0.5) (layer "B.Cu") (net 30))
 (segment (start 78.2 128.2) (end 96.59 128.2) (width 0.5) (layer "B.Cu") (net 30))
 (segment (start 77.2 34.4) (end 77.2 84.7) (width 0.5) (layer "B.Cu") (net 30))
 (segment (start 80.359022 107.84) (end 77.76 107.84) (width 0.5) (layer "B.Cu") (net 30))
 (segment (start 77.76 107.84) (end 77.5 108.1) (width 0.5) (layer "B.Cu") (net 30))
 (segment (start 83 105.199022) (end 80.359022 107.84) (width 0.5) (layer "B.Cu") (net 30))
 (segment (start 79.81 86.5) (end 80.01 86.3) (width 0.5) (layer "B.Cu") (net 30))
 (segment (start 105.41 71.12) (end 86.3 52.01) (width 0.5) (layer "B.Cu") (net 30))
 (segment (start 86.3 52.01) (end 86.3 33.5) (width 0.5) (layer "B.Cu") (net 30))
 (segment (start 84.5 31.7) (end 79.9 31.7) (width 0.5) (layer "B.Cu") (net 30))
 (segment (start 106.5 71.12) (end 105.41 71.12) (width 0.5) (layer "B.Cu") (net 30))
 (segment (start 77.5 127.5) (end 78.2 128.2) (width 0.5) (layer "B.Cu") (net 30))
 (segment (start 86.3 33.5) (end 84.5 31.7) (width 0.5) (layer "B.Cu") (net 30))
 (segment (start 123.9 88.52) (end 106.5 71.12) (width 0.5) (layer "B.Cu") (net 30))
 (segment (start 79 86.5) (end 79.81 86.5) (width 0.5) (layer "B.Cu") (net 30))
 (segment (start 80.01 88.84) (end 83 91.83) (width 0.5) (layer "B.Cu") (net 30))
 (segment (start 83 91.83) (end 83 105.199022) (width 0.5) (layer "B.Cu") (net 30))
 (segment (start 80.01 86.3) (end 80.01 88.84) (width 0.5) (layer "B.Cu") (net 30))
 (segment (start 77.2 84.7) (end 79 86.5) (width 0.5) (layer "B.Cu") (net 30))
 (segment (start 86.7 114.3) (end 97.79 114.3) (width 0.5) (layer "B.Cu") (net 65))
 (segment (start 80.3 110.38) (end 82.78 110.38) (width 0.5) (layer "B.Cu") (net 65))
 (segment (start 82.78 110.38) (end 86.7 114.3) (width 0.5) (layer "B.Cu") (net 65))
 (segment (start 86.74 116.84) (end 97.79 116.84) (width 0.5) (layer "B.Cu") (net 66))
 (segment (start 80.3 112.92) (end 82.82 112.92) (width 0.5) (layer "B.Cu") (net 66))
 (segment (start 82.82 112.92) (end 86.74 116.84) (width 0.5) (layer "B.Cu") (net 66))
 (segment (start 80.3 119.62) (end 97.55 119.62) (width 0.5) (layer "B.Cu") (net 50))
 (segment (start 97.55 119.62) (end 97.79 119.38) (width 0.5) (layer "B.Cu") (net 50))
 (segment (start 97.55 122.16) (end 97.79 121.92) (width 0.5) (layer "B.Cu") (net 51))
 (segment (start 80.3 122.16) (end 97.55 122.16) (width 0.5) (layer "B.Cu") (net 51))
 (segment (start 97.536 122.174) (end 97.79 121.92) (width 0.25) (layer "B.Cu") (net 51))
 (segment (start 97.55 124.7) (end 97.79 124.46) (width 0.5) (layer "B.Cu") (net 52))
 (segment (start 80.3 124.7) (end 97.55 124.7) (width 0.5) (layer "B.Cu") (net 52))
 (segment (start 112.94 104.14) (end 114.3 104.14) (width 0.5) (layer "B.Cu") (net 6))
 (segment (start 102.6 93.8) (end 112.94 104.14) (width 0.5) (layer "B.Cu") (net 6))
 (segment (start 102.6 69.58) (end 102.6 93.8) (width 0.5) (layer "B.Cu") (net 6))
 (segment (start 81.28 48.26) (end 82.55 48.26) (width 0.25) (layer "B.Cu") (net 6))
 (segment (start 81.28 48.26) (end 102.6 69.58) (width 0.5) (layer "B.Cu") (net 6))
 (segment (start 98.230992 67.750992) (end 98.250992 67.750992) (width 0.5) (layer "B.Cu") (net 7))
 (segment (start 81.28 50.8) (end 98.230992 67.750992) (width 0.5) (layer "B.Cu") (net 7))
 (segment (start 98.250992 67.750992) (end 101 70.5) (width 0.5) (layer "B.Cu") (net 7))
 (segment (start 101 95) (end 112.68 106.68) (width 0.5) (layer "B.Cu") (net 7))
 (segment (start 112.68 106.68) (end 114.3 106.68) (width 0.5) (layer "B.Cu") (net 7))
 (segment (start 101 70.5) (end 101 95) (width 0.5) (layer "B.Cu") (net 7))
 (segment (start 115.9 99.06) (end 123.9 91.06) (width 0.5) (layer "B.Cu") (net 38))
 (segment (start 114.3 99.06) (end 115.9 99.06) (width 0.5) (layer "B.Cu") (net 38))
 (segment (start 114.3 99.06) (end 115.57 99.06) (width 0.5) (layer "B.Cu") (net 38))
 (segment (start 121.3 46.6) (end 121.4 46.5) (width 0.9) (layer "B.Cu") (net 31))
 (segment (start 121.3 55.4) (end 121.3 46.6) (width 0.9) (layer "B.Cu") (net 31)))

